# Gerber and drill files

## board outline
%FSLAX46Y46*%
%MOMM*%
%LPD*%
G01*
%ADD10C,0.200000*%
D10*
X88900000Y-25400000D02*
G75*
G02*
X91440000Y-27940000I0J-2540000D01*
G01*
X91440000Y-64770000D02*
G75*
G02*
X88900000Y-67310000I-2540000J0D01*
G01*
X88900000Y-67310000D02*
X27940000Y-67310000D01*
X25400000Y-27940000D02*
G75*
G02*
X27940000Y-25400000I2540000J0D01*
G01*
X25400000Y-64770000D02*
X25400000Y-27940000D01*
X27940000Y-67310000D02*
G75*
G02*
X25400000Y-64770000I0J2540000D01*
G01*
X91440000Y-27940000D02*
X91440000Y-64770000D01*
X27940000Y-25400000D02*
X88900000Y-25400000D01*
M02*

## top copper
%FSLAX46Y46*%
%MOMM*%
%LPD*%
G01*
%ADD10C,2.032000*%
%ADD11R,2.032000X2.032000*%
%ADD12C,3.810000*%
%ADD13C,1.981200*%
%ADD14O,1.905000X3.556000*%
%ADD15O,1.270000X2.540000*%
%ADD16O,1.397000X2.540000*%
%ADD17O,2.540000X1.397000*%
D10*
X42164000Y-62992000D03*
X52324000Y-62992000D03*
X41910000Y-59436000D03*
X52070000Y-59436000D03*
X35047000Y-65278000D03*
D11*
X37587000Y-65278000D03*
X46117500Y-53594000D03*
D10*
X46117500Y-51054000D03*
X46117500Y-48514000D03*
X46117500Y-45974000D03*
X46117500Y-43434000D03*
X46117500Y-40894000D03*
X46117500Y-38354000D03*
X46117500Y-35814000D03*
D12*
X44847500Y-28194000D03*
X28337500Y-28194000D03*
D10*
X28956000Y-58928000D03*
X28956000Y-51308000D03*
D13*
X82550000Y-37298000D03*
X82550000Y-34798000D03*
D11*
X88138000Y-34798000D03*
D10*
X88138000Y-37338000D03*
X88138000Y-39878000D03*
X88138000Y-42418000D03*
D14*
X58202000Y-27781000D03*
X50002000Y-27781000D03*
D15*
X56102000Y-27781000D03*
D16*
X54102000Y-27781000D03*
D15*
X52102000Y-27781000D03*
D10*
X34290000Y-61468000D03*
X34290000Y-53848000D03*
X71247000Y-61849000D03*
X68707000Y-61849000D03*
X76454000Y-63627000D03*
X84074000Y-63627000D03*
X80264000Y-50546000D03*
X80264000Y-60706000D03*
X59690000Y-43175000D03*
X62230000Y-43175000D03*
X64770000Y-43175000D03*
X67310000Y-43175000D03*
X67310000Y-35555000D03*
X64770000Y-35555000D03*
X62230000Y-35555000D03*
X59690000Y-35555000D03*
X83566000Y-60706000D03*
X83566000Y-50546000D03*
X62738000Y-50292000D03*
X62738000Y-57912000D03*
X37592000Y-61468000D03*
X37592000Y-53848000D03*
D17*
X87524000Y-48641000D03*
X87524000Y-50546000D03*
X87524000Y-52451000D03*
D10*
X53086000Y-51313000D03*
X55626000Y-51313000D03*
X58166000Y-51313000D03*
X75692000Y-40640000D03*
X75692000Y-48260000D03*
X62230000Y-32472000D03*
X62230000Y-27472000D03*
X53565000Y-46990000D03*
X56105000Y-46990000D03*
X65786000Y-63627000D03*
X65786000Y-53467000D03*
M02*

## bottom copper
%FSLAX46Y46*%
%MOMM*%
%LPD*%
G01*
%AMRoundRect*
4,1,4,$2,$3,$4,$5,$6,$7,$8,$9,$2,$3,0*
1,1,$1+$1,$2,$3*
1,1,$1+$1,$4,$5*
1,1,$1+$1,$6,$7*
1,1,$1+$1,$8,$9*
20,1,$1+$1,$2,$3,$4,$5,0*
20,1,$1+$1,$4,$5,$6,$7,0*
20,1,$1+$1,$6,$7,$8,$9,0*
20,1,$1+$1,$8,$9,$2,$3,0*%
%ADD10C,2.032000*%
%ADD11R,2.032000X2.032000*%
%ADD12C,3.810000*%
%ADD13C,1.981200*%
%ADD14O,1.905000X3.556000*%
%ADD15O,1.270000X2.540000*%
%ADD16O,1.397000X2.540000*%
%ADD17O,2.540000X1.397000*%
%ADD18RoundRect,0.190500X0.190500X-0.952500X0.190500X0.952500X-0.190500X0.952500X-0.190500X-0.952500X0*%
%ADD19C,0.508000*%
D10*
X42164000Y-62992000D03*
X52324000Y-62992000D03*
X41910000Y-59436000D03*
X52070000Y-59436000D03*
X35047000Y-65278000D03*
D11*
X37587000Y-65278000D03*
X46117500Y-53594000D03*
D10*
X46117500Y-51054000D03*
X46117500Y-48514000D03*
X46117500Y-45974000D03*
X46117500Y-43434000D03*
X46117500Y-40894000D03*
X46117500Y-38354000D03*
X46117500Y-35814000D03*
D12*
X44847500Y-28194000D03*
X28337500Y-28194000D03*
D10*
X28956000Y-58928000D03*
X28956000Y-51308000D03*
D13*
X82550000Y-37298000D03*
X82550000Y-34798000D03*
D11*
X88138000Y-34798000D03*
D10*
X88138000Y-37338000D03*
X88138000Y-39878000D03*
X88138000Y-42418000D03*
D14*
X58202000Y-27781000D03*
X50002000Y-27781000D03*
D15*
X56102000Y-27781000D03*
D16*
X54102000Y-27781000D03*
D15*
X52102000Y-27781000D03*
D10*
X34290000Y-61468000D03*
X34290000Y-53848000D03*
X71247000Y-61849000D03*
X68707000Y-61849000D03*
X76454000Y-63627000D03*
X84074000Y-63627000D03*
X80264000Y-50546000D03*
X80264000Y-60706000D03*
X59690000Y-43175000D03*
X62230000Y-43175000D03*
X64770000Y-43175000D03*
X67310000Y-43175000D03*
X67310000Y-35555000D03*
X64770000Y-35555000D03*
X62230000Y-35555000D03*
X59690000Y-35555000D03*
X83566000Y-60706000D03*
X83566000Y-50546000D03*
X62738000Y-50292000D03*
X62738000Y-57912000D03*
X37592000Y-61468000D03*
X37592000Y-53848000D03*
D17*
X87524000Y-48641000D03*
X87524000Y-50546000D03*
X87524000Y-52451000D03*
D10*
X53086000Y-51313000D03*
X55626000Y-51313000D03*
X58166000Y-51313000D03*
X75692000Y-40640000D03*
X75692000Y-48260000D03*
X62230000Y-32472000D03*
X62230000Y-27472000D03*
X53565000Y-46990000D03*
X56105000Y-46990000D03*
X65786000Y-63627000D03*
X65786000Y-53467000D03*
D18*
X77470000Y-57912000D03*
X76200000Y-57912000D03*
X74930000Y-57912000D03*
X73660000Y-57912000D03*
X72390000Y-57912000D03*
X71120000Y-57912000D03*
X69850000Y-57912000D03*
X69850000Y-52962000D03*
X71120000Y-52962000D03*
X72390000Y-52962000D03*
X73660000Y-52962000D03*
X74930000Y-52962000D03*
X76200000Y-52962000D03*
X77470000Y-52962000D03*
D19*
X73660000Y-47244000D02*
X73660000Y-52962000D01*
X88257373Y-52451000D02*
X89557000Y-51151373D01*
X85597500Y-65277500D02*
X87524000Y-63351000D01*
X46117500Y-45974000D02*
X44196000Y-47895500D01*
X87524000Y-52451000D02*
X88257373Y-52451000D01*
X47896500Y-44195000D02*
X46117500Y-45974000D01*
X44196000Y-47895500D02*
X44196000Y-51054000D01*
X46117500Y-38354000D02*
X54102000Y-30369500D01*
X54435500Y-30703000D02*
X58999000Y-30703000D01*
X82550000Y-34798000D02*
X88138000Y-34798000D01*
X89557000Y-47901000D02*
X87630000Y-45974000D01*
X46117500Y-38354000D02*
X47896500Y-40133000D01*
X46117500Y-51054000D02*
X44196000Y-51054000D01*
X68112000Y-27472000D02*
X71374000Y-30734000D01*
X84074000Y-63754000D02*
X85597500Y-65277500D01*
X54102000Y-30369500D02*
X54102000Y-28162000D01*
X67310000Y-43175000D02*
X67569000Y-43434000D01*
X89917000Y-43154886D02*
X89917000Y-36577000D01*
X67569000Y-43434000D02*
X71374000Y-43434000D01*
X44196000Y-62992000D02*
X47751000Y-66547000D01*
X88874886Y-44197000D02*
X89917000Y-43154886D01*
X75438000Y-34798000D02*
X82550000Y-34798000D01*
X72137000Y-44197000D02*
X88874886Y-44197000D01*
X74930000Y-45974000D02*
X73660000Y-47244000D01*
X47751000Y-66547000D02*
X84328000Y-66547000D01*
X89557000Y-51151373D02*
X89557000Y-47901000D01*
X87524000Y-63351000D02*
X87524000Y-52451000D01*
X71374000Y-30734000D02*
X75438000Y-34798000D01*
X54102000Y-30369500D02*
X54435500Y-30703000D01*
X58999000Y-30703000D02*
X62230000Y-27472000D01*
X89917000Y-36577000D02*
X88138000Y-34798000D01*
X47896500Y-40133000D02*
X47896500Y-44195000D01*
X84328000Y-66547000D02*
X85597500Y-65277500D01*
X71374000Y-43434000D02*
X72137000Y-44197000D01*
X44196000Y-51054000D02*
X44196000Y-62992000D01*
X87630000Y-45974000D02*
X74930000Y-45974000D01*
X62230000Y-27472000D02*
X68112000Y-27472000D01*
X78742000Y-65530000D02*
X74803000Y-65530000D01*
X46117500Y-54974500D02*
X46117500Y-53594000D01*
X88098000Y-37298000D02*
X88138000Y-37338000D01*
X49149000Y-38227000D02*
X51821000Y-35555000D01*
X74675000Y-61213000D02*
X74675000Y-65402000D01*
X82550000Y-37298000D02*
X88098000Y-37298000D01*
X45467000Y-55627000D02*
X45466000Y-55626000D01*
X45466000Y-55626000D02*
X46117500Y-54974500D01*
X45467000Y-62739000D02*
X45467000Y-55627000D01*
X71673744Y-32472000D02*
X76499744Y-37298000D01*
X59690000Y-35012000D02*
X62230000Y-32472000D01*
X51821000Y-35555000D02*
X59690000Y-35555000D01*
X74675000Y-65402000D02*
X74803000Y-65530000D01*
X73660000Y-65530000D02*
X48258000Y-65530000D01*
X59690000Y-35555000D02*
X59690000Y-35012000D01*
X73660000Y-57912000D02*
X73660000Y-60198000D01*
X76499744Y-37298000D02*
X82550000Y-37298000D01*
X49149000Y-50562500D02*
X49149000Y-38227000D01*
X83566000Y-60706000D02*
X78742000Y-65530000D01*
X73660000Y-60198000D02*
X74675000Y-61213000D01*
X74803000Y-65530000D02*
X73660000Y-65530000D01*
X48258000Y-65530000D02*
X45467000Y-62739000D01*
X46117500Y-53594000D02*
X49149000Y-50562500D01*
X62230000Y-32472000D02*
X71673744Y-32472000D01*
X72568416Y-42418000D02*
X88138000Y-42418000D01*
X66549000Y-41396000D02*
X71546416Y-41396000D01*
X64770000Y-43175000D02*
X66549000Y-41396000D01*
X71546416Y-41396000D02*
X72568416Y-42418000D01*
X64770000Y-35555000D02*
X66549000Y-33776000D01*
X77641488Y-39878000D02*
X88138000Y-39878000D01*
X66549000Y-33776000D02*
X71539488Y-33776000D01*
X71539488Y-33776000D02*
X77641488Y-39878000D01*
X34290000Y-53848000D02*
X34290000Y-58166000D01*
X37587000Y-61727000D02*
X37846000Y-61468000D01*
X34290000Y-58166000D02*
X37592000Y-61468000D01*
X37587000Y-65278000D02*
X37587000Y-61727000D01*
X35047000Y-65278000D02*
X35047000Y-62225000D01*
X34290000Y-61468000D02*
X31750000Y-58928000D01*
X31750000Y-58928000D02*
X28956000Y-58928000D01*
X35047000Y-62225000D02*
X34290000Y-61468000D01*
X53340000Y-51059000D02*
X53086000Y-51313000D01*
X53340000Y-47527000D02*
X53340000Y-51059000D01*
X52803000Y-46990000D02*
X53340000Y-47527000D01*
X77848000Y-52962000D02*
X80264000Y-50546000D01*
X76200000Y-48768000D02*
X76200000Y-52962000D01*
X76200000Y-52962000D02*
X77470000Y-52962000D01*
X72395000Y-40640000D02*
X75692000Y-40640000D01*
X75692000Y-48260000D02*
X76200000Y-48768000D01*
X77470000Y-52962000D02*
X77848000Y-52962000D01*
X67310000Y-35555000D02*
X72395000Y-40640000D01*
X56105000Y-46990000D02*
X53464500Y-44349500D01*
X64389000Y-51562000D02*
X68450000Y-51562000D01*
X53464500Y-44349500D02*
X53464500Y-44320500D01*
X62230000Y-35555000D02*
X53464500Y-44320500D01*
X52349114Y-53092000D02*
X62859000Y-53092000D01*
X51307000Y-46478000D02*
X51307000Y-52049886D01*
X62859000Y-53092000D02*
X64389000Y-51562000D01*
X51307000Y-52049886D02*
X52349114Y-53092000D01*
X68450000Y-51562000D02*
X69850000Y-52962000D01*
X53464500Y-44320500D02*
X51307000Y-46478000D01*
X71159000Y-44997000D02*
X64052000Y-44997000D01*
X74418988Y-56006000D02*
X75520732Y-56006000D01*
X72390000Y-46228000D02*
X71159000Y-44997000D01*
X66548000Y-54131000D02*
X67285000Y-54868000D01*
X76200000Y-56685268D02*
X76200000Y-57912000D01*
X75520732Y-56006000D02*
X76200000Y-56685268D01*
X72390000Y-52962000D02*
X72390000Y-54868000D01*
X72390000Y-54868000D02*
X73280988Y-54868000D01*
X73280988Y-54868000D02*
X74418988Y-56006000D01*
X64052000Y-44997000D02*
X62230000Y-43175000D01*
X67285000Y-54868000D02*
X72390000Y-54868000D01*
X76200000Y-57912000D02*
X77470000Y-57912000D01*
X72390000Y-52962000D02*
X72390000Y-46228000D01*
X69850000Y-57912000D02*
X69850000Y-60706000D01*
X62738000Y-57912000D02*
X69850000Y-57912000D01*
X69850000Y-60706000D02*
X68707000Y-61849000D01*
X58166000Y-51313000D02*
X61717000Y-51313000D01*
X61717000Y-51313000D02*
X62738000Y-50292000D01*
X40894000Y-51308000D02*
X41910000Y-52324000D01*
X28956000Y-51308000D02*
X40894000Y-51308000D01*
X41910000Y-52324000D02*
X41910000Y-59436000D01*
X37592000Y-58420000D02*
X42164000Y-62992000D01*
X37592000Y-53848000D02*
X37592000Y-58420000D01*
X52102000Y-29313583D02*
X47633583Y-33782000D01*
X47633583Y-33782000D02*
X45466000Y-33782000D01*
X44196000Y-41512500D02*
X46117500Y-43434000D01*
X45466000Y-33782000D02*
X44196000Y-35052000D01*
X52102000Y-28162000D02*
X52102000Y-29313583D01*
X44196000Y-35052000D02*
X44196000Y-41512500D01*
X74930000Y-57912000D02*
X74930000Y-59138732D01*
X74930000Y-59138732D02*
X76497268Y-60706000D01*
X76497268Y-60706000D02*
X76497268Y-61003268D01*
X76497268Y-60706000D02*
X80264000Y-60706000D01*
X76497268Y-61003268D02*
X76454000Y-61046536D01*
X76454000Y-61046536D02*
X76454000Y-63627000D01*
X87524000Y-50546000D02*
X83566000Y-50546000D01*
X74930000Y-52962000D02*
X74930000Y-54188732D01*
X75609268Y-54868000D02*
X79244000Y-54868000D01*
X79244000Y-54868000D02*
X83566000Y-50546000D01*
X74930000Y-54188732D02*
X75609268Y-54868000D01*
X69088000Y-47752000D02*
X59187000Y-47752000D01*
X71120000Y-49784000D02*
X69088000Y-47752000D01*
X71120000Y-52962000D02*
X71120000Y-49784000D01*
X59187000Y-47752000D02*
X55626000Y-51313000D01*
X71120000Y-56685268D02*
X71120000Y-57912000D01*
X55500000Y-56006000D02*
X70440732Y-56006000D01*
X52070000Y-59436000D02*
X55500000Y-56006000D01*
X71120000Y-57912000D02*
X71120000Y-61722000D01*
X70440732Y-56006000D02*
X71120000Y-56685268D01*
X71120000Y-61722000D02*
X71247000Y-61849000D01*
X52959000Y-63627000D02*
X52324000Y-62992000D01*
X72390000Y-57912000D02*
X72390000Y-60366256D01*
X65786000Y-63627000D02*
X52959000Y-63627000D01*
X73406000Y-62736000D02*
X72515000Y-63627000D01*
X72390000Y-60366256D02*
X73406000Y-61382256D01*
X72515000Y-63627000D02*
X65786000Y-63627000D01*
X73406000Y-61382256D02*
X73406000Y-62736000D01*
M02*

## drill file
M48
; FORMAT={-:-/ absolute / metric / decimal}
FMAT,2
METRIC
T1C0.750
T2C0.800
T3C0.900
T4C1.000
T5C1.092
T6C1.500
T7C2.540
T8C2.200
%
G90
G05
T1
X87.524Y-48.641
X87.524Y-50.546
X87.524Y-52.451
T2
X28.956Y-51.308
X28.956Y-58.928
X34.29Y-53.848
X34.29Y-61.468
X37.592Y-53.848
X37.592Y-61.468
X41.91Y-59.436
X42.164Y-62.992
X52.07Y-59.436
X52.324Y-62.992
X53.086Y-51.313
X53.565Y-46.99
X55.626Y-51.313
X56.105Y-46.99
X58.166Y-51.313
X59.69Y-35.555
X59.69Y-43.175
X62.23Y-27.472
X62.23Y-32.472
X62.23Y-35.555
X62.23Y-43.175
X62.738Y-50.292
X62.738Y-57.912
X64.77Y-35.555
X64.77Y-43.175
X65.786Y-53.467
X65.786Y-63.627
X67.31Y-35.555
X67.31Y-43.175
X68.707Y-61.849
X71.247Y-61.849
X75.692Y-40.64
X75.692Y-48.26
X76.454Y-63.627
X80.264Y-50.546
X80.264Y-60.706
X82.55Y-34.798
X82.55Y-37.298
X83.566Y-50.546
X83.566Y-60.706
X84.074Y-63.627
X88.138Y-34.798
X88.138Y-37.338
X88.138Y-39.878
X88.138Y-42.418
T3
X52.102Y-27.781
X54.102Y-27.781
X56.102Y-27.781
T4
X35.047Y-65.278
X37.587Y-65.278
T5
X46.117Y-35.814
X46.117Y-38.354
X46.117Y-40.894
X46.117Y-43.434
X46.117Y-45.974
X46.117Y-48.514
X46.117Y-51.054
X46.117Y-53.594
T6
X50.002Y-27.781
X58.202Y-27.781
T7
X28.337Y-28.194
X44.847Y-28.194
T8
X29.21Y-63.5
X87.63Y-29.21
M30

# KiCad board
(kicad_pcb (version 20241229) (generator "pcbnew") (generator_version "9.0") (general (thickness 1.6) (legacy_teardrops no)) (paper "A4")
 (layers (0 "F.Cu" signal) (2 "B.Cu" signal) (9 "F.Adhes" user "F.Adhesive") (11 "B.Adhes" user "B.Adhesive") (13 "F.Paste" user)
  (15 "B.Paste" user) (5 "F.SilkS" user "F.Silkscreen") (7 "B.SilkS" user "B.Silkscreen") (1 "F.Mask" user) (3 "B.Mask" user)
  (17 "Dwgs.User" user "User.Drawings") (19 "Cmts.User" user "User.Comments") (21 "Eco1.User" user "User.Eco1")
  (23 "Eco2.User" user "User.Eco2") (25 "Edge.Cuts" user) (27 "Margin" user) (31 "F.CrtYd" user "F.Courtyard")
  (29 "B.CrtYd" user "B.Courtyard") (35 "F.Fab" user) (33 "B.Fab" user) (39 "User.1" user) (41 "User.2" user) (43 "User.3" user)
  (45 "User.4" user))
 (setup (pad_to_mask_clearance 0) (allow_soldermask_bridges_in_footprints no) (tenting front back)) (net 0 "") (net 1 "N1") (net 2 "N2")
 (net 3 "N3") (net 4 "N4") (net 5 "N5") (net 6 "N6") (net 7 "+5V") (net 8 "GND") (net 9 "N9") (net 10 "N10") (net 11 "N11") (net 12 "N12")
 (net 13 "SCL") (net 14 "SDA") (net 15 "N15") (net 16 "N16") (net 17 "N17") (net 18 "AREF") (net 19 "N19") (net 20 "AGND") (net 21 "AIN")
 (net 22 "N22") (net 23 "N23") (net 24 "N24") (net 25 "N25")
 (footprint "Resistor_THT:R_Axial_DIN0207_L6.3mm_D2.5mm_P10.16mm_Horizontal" (layer "F.Cu") (at 42.164 62.992)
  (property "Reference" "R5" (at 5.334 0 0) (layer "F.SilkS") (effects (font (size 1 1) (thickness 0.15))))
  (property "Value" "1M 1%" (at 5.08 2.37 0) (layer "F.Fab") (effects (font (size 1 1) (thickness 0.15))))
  (pad "1" thru_hole circle (at 0 0) (size 2.032 2.032) (drill 0.8) (layers "*.Cu" "*.Mask") (remove_unused_layers no) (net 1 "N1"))
  (pad "2" thru_hole circle (at 10.16 0) (size 2.032 2.032) (drill 0.8) (layers "*.Cu" "*.Mask") (remove_unused_layers no) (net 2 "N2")))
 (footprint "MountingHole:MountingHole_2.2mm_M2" (layer "F.Cu") (at 29.21 63.5)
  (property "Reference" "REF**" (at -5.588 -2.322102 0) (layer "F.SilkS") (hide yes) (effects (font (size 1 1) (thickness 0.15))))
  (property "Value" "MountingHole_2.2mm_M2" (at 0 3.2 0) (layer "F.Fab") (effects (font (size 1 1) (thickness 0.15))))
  (pad "" np_thru_hole circle (at 0 0) (size 2.2 2.2) (drill 2.2) (layers "*.Cu" "*.Mask")))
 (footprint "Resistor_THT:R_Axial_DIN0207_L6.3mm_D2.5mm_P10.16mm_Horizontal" (layer "F.Cu") (at 41.91 59.436)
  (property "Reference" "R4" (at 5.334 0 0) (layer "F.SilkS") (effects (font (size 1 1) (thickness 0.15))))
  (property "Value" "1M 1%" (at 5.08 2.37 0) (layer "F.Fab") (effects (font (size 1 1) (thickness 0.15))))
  (pad "1" thru_hole circle (at 0 0) (size 2.032 2.032) (drill 0.8) (layers "*.Cu" "*.Mask") (remove_unused_layers no) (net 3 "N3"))
  (pad "2" thru_hole circle (at 10.16 0) (size 2.032 2.032) (drill 0.8) (layers "*.Cu" "*.Mask") (remove_unused_layers no) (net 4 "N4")))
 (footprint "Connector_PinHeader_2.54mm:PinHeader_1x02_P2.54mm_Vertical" (layer "F.Cu") (at 35.047 65.278 90)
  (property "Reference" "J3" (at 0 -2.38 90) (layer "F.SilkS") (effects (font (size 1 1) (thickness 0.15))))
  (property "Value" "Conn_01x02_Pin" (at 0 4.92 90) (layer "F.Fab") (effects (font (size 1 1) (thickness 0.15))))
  (pad "1" thru_hole circle (at 0 0 90) (size 2.032 2.032) (drill 1) (layers "*.Cu" "*.Mask") (remove_unused_layers no) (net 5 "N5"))
  (pad "2" thru_hole rect (at 0 2.54 90) (size 2.032 2.032) (drill 1) (layers "*.Cu" "*.Mask") (remove_unused_layers no) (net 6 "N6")))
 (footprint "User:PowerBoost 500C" (layer "F.Cu") (at 46.1175 53.594 180)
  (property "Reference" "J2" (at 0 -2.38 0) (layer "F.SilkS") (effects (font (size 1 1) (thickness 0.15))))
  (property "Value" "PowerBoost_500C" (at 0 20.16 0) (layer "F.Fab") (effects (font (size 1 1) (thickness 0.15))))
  (pad "1" thru_hole rect (at 0 0 180) (size 2.032 2.032) (drill 1.0922) (layers "*.Cu" "*.Mask") (remove_unused_layers no) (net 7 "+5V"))
  (pad "2" thru_hole circle (at 0 2.54 180) (size 2.032 2.032) (drill 1.0922) (layers "*.Cu" "*.Mask") (remove_unused_layers no)
   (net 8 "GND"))
  (pad "3" thru_hole circle (at 0 5.08 180) (size 2.032 2.032) (drill 1.0922) (layers "*.Cu" "*.Mask") (remove_unused_layers no)
   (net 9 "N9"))
  (pad "4" thru_hole circle (at 0 7.62 180) (size 2.032 2.032) (drill 1.0922) (layers "*.Cu" "*.Mask") (remove_unused_layers no)
   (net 8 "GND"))
  (pad "5" thru_hole circle (at 0 10.16 180) (size 2.032 2.032) (drill 1.0922) (layers "*.Cu" "*.Mask") (remove_unused_layers no)
   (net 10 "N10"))
  (pad "6" thru_hole circle (at 0 12.7 180) (size 2.032 2.032) (drill 1.0922) (layers "*.Cu" "*.Mask") (remove_unused_layers no)
   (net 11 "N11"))
  (pad "7" thru_hole circle (at 0 15.24 180) (size 2.032 2.032) (drill 1.0922) (layers "*.Cu" "*.Mask") (remove_unused_layers no)
   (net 8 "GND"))
  (pad "8" thru_hole circle (at 0 17.78 180) (size 2.032 2.032) (drill 1.0922) (layers "*.Cu" "*.Mask") (remove_unused_layers no)
   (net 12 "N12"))
  (pad "9" thru_hole circle (at 1.27 25.4 180) (size 3.81 3.81) (drill 2.54) (layers "*.Cu" "*.Mask") (remove_unused_layers no))
  (pad "9" thru_hole circle (at 17.78 25.4 180) (size 3.81 3.81) (drill 2.54) (layers "*.Cu" "*.Mask") (remove_unused_layers no)))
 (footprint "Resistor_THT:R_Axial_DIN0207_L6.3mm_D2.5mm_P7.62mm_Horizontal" (layer "F.Cu") (at 28.956 58.928 90)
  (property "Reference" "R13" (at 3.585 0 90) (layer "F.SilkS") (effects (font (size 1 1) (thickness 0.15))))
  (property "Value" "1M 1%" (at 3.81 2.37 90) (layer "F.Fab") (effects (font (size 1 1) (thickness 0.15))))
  (pad "1" thru_hole circle (at 0 0 90) (size 2.032 2.032) (drill 0.8) (layers "*.Cu" "*.Mask") (remove_unused_layers no) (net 5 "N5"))
  (pad "2" thru_hole circle (at 7.62 0 90) (size 2.032 2.032) (drill 0.8) (layers "*.Cu" "*.Mask") (remove_unused_layers no) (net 3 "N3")))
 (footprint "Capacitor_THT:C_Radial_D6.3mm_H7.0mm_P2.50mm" (layer "F.Cu") (at 82.55 37.298 90)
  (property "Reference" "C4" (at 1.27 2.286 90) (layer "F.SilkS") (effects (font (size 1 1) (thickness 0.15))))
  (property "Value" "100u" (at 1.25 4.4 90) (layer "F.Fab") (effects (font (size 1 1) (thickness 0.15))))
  (pad "1" thru_hole circle (at 0 0 90) (size 1.9812 1.9812) (drill 0.8) (layers "*.Cu" "*.Mask") (remove_unused_layers no) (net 7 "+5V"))
  (pad "2" thru_hole circle (at 2.5 0 90) (size 1.9812 1.9812) (drill 0.8) (layers "*.Cu" "*.Mask") (remove_unused_layers no) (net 8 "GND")))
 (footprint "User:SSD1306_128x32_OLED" (layer "F.Cu") (at 88.138 34.798)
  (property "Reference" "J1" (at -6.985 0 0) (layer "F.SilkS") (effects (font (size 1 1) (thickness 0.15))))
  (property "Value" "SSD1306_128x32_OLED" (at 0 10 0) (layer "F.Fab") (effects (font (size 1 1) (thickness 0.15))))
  (pad "1" thru_hole rect (at 0 0) (size 2.032 2.032) (drill 0.8) (layers "*.Cu" "*.Mask") (remove_unused_layers no) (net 8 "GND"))
  (pad "2" thru_hole circle (at 0 2.54) (size 2.032 2.032) (drill 0.8) (layers "*.Cu" "*.Mask") (remove_unused_layers no) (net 7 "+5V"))
  (pad "3" thru_hole circle (at 0 5.08) (size 2.032 2.032) (drill 0.8) (layers "*.Cu" "*.Mask") (remove_unused_layers no) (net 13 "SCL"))
  (pad "4" thru_hole circle (at 0 7.62) (size 2.032 2.032) (drill 0.8) (layers "*.Cu" "*.Mask") (remove_unused_layers no) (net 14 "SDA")))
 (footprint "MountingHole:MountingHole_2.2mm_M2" (layer "F.Cu") (at 87.63 29.21)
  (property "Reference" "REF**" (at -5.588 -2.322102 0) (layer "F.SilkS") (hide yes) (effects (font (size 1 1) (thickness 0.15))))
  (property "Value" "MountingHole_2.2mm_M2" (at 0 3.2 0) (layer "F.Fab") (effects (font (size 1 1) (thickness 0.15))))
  (pad "" np_thru_hole circle (at 0 0) (size 2.2 2.2) (drill 2.2) (layers "*.Cu" "*.Mask")))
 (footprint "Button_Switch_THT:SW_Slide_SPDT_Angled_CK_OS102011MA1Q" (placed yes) (layer "F.Cu") (at 56.102 27.781 180)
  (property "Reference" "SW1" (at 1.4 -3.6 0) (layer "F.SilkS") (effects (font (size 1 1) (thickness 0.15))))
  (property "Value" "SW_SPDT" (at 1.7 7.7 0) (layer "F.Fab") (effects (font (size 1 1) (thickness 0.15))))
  (pad "" thru_hole oval (at -2.1 0 180) (size 1.905 3.556) (drill 1.5) (layers "*.Cu" "*.Mask") (remove_unused_layers no))
  (pad "" thru_hole oval (at 6.1 0 180) (size 1.905 3.556) (drill 1.5) (layers "*.Cu" "*.Mask") (remove_unused_layers no))
  (pad "1" thru_hole oval (at 0 0 180) (size 1.27 2.54) (drill 0.9) (layers "*.Cu" "*.Mask") (remove_unused_layers no) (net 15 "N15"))
  (pad "2" thru_hole oval (at 2 0 180) (size 1.397 2.54) (drill 0.9) (layers "*.Cu" "*.Mask") (remove_unused_layers no) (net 8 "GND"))
  (pad "3" thru_hole oval (at 4 0 180) (size 1.27 2.54) (drill 0.9) (layers "*.Cu" "*.Mask") (remove_unused_layers no) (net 10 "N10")))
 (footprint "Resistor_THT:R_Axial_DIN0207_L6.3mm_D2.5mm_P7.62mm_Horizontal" (layer "F.Cu") (at 34.29 61.468 90)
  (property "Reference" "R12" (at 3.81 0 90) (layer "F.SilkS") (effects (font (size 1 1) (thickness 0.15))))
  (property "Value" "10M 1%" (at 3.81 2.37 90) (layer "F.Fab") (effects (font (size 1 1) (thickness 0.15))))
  (pad "1" thru_hole circle (at 0 0 90) (size 2.032 2.032) (drill 0.8) (layers "*.Cu" "*.Mask") (remove_unused_layers no) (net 5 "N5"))
  (pad "2" thru_hole circle (at 7.62 0 90) (size 2.032 2.032) (drill 0.8) (layers "*.Cu" "*.Mask") (remove_unused_layers no) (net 6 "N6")))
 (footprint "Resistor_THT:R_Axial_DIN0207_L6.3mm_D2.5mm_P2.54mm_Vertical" (layer "F.Cu") (at 71.247 61.849 180)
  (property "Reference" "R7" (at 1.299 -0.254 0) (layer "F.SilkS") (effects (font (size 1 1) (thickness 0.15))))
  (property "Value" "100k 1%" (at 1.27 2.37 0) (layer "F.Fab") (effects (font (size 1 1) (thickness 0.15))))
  (pad "1" thru_hole circle (at 0 0 180) (size 2.032 2.032) (drill 0.8) (layers "*.Cu" "*.Mask") (remove_unused_layers no) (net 4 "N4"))
  (pad "2" thru_hole circle (at 2.54 0 180) (size 2.032 2.032) (drill 0.8) (layers "*.Cu" "*.Mask") (remove_unused_layers no) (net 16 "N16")))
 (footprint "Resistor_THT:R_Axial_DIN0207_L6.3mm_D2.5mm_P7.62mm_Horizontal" (layer "F.Cu") (at 76.454 63.627)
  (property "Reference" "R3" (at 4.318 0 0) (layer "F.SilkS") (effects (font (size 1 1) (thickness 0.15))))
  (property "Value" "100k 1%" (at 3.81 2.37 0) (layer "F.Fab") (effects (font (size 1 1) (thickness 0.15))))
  (pad "1" thru_hole circle (at 0 0) (size 2.032 2.032) (drill 0.8) (layers "*.Cu" "*.Mask") (remove_unused_layers no) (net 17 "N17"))
  (pad "2" thru_hole circle (at 7.62 0) (size 2.032 2.032) (drill 0.8) (layers "*.Cu" "*.Mask") (remove_unused_layers no) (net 8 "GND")))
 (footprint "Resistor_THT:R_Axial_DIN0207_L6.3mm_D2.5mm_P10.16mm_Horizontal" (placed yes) (layer "F.Cu") (at 80.264 50.546 -90)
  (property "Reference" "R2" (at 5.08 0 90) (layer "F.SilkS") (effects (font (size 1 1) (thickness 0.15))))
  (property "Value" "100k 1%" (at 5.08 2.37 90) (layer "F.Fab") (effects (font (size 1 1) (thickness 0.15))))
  (pad "1" thru_hole circle (at 0 0 270) (size 2.032 2.032) (drill 0.8) (layers "*.Cu" "*.Mask") (remove_unused_layers no) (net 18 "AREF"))
  (pad "2" thru_hole circle (at 10.16 0 270) (size 2.032 2.032) (drill 0.8) (layers "*.Cu" "*.Mask") (remove_unused_layers no)
   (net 17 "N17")))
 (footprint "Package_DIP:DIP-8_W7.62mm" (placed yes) (layer "F.Cu") (at 59.69 43.175 90)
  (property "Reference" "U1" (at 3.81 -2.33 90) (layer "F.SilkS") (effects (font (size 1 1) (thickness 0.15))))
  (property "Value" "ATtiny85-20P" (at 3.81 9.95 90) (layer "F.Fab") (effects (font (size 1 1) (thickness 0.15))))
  (pad "1" thru_hole circle (at 0 0 90) (size 2.032 2.032) (drill 0.8) (layers "*.Cu" "*.Mask") (remove_unused_layers no) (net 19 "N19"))
  (pad "2" thru_hole circle (at 0 2.54 90) (size 2.032 2.032) (drill 0.8) (layers "*.Cu" "*.Mask") (remove_unused_layers no) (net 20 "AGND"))
  (pad "3" thru_hole circle (at 0 5.08 90) (size 2.032 2.032) (drill 0.8) (layers "*.Cu" "*.Mask") (remove_unused_layers no) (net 14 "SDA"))
  (pad "4" thru_hole circle (at 0 7.62 90) (size 2.032 2.032) (drill 0.8) (layers "*.Cu" "*.Mask") (remove_unused_layers no) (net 8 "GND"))
  (pad "5" thru_hole circle (at 7.62 7.62 90) (size 2.032 2.032) (drill 0.8) (layers "*.Cu" "*.Mask") (remove_unused_layers no)
   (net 18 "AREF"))
  (pad "6" thru_hole circle (at 7.62 5.08 90) (size 2.032 2.032) (drill 0.8) (layers "*.Cu" "*.Mask") (remove_unused_layers no)
   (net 13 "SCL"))
  (pad "7" thru_hole circle (at 7.62 2.54 90) (size 2.032 2.032) (drill 0.8) (layers "*.Cu" "*.Mask") (remove_unused_layers no)
   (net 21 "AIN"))
  (pad "8" thru_hole circle (at 7.62 0 90) (size 2.032 2.032) (drill 0.8) (layers "*.Cu" "*.Mask") (remove_unused_layers no) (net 7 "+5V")))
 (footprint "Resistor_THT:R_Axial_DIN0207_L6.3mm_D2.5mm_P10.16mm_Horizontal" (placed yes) (layer "F.Cu") (at 83.566 60.706 90)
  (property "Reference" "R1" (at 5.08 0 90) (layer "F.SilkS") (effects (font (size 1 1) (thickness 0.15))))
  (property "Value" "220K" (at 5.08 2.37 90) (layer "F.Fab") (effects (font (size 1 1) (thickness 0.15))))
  (pad "1" thru_hole circle (at 0 0 90) (size 2.032 2.032) (drill 0.8) (layers "*.Cu" "*.Mask") (remove_unused_layers no) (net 7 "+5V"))
  (pad "2" thru_hole circle (at 10.16 0 90) (size 2.032 2.032) (drill 0.8) (layers "*.Cu" "*.Mask") (remove_unused_layers no) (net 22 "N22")))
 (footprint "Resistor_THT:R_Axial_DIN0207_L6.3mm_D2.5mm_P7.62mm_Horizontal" (layer "F.Cu") (at 62.738 50.292 -90)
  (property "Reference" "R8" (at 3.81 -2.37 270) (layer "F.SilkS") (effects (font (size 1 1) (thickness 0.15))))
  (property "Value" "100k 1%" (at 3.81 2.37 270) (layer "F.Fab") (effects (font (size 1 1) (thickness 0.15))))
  (pad "1" thru_hole circle (at 0 0 270) (size 2.032 2.032) (drill 0.8) (layers "*.Cu" "*.Mask") (remove_unused_layers no) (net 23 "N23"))
  (pad "2" thru_hole circle (at 7.62 0 270) (size 2.032 2.032) (drill 0.8) (layers "*.Cu" "*.Mask") (remove_unused_layers no) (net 16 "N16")))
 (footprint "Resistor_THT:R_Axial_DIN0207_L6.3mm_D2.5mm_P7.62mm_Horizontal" (layer "F.Cu") (at 37.592 61.468 90)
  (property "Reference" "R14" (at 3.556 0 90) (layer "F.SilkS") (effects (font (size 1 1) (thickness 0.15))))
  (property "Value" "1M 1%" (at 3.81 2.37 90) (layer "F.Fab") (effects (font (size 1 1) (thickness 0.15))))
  (pad "1" thru_hole circle (at 0 0 90) (size 2.032 2.032) (drill 0.8) (layers "*.Cu" "*.Mask") (remove_unused_layers no) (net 6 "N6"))
  (pad "2" thru_hole circle (at 7.62 0 90) (size 2.032 2.032) (drill 0.8) (layers "*.Cu" "*.Mask") (remove_unused_layers no) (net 1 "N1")))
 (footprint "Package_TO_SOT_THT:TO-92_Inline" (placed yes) (layer "F.Cu") (at 87.524 49.276 -90)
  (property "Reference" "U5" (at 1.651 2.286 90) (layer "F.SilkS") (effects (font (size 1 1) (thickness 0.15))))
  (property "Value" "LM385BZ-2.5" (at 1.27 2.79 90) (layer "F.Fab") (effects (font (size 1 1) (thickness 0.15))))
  (pad "1" thru_hole oval (at -0.635 0 270) (size 1.397 2.54) (drill 0.75) (layers "*.Cu" "*.Mask") (remove_unused_layers no))
  (pad "2" thru_hole oval (at 1.27 0 270) (size 1.397 2.54) (drill 0.75) (layers "*.Cu" "*.Mask") (remove_unused_layers no) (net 22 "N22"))
  (pad "3" thru_hole oval (at 3.175 0 270) (size 1.397 2.54) (drill 0.75) (layers "*.Cu" "*.Mask") (remove_unused_layers no) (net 8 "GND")))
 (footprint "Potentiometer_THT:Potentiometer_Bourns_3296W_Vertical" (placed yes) (layer "F.Cu") (at 53.086 51.313 180)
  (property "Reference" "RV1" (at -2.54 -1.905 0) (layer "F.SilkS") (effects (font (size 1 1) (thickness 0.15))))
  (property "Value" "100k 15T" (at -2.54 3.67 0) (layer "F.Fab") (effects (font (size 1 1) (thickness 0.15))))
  (pad "1" thru_hole circle (at 0 0 180) (size 2.032 2.032) (drill 0.8) (layers "*.Cu" "*.Mask") (remove_unused_layers no) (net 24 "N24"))
  (pad "2" thru_hole circle (at -2.54 0 180) (size 2.032 2.032) (drill 0.8) (layers "*.Cu" "*.Mask") (remove_unused_layers no)
   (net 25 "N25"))
  (pad "3" thru_hole circle (at -5.08 0 180) (size 2.032 2.032) (drill 0.8) (layers "*.Cu" "*.Mask") (remove_unused_layers no)
   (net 23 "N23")))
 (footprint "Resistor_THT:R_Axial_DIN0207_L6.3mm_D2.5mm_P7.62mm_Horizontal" (layer "F.Cu") (at 75.692 40.64 -90)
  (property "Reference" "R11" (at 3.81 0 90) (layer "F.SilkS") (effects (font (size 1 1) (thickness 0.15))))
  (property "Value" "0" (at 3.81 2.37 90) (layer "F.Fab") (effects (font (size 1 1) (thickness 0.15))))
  (pad "1" thru_hole circle (at 0 0 270) (size 2.032 2.032) (drill 0.8) (layers "*.Cu" "*.Mask") (remove_unused_layers no) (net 18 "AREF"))
  (pad "2" thru_hole circle (at 7.62 0 270) (size 2.032 2.032) (drill 0.8) (layers "*.Cu" "*.Mask") (remove_unused_layers no)
   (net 18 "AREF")))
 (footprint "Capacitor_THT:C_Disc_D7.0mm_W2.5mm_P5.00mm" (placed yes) (layer "F.Cu") (at 62.23 32.472 90)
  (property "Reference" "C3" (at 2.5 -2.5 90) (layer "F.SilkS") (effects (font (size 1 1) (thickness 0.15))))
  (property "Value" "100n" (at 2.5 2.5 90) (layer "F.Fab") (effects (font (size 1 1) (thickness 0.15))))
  (pad "1" thru_hole circle (at 0 0 90) (size 2.032 2.032) (drill 0.8) (layers "*.Cu" "*.Mask") (remove_unused_layers no) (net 7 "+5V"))
  (pad "2" thru_hole circle (at 5 0 90) (size 2.032 2.032) (drill 0.8) (layers "*.Cu" "*.Mask") (remove_unused_layers no) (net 8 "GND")))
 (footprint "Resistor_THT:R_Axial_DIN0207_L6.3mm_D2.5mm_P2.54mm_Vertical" (layer "F.Cu") (at 53.565 46.99)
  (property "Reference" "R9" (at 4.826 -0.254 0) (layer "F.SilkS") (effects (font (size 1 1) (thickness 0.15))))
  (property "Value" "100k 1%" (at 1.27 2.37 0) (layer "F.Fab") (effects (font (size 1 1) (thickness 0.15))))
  (pad "1" thru_hole circle (at 0 0) (size 2.032 2.032) (drill 0.8) (layers "*.Cu" "*.Mask") (remove_unused_layers no) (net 24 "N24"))
  (pad "2" thru_hole circle (at 2.54 0) (size 2.032 2.032) (drill 0.8) (layers "*.Cu" "*.Mask") (remove_unused_layers no) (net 21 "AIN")))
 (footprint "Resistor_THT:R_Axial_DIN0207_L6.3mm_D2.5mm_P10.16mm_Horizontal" (layer "F.Cu") (at 65.786 63.627 90)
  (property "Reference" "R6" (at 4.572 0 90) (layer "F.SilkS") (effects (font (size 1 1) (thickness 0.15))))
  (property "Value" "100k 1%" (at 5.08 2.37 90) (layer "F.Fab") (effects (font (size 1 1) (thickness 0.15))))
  (pad "1" thru_hole circle (at 0 0 90) (size 2.032 2.032) (drill 0.8) (layers "*.Cu" "*.Mask") (remove_unused_layers no) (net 2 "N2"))
  (pad "2" thru_hole circle (at 10.16 0 90) (size 2.032 2.032) (drill 0.8) (layers "*.Cu" "*.Mask") (remove_unused_layers no)
   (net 20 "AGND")))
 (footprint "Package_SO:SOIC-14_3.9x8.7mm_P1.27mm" (layer "B.Cu") (at 73.66 55.437 90)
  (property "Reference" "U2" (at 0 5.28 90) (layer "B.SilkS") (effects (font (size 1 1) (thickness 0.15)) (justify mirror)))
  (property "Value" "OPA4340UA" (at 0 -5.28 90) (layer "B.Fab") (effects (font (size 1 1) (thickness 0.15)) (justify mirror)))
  (pad "1" smd roundrect (at -2.475 3.81 90) (size 2.286 0.762) (layers "B.Cu" "B.Mask" "B.Paste") (roundrect_rratio 0.25) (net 20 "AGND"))
  (pad "2" smd roundrect (at -2.475 2.54 90) (size 2.286 0.762) (layers "B.Cu" "B.Mask" "B.Paste") (roundrect_rratio 0.25) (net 20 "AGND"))
  (pad "3" smd roundrect (at -2.475 1.27 90) (size 2.286 0.762) (layers "B.Cu" "B.Mask" "B.Paste") (roundrect_rratio 0.25) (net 17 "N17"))
  (pad "4" smd roundrect (at -2.475 0 90) (size 2.286 0.762) (layers "B.Cu" "B.Mask" "B.Paste") (roundrect_rratio 0.25) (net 7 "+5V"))
  (pad "5" smd roundrect (at -2.475 -1.27 90) (size 2.286 0.762) (layers "B.Cu" "B.Mask" "B.Paste") (roundrect_rratio 0.25) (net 2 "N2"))
  (pad "6" smd roundrect (at -2.475 -2.54 90) (size 2.286 0.762) (layers "B.Cu" "B.Mask" "B.Paste") (roundrect_rratio 0.25) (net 4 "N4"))
  (pad "7" smd roundrect (at -2.475 -3.81 90) (size 2.286 0.762) (layers "B.Cu" "B.Mask" "B.Paste") (roundrect_rratio 0.25) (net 16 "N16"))
  (pad "8" smd roundrect (at 2.475 -3.81 90) (size 2.286 0.762) (layers "B.Cu" "B.Mask" "B.Paste") (roundrect_rratio 0.25) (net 21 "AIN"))
  (pad "9" smd roundrect (at 2.475 -2.54 90) (size 2.286 0.762) (layers "B.Cu" "B.Mask" "B.Paste") (roundrect_rratio 0.25) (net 25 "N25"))
  (pad "10" smd roundrect (at 2.475 -1.27 90) (size 2.286 0.762) (layers "B.Cu" "B.Mask" "B.Paste") (roundrect_rratio 0.25) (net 20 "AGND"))
  (pad "11" smd roundrect (at 2.475 0 90) (size 2.286 0.762) (layers "B.Cu" "B.Mask" "B.Paste") (roundrect_rratio 0.25) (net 8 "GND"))
  (pad "12" smd roundrect (at 2.475 1.27 90) (size 2.286 0.762) (layers "B.Cu" "B.Mask" "B.Paste") (roundrect_rratio 0.25) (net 22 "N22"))
  (pad "13" smd roundrect (at 2.475 2.54 90) (size 2.286 0.762) (layers "B.Cu" "B.Mask" "B.Paste") (roundrect_rratio 0.25) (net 18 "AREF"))
  (pad "14" smd roundrect (at 2.475 3.81 90) (size 2.286 0.762) (layers "B.Cu" "B.Mask" "B.Paste") (roundrect_rratio 0.25) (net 18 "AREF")))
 (gr_arc (start 88.9 25.4) (mid 90.696051 26.143949) (end 91.44 27.94) (stroke (width 0.2) (type default)) (layer "Edge.Cuts"))
 (gr_arc (start 91.44 64.77) (mid 90.696051 66.566051) (end 88.9 67.31) (stroke (width 0.2) (type default)) (layer "Edge.Cuts"))
 (gr_line (start 88.9 67.31) (end 27.94 67.31) (stroke (width 0.2) (type default)) (layer "Edge.Cuts"))
 (gr_arc (start 25.4 27.94) (mid 26.143949 26.143949) (end 27.94 25.4) (stroke (width 0.2) (type default)) (layer "Edge.Cuts"))
 (gr_line (start 25.4 64.77) (end 25.4 27.94) (stroke (width 0.2) (type default)) (layer "Edge.Cuts"))
 (gr_arc (start 27.94 67.31) (mid 26.143949 66.566051) (end 25.4 64.77) (stroke (width 0.2) (type default)) (layer "Edge.Cuts"))
 (gr_line (start 91.44 27.94) (end 91.44 64.77) (stroke (width 0.2) (type default)) (layer "Edge.Cuts"))
 (gr_line (start 27.94 25.4) (end 88.9 25.4) (stroke (width 0.2) (type default)) (layer "Edge.Cuts"))
 (segment (start 73.66 47.244) (end 73.66 52.962) (width 0.508) (layer "B.Cu") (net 8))
 (segment (start 88.257373 52.451) (end 89.557 51.151373) (width 0.508) (layer "B.Cu") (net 8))
 (segment (start 85.5975 65.2775) (end 87.524 63.351) (width 0.508) (layer "B.Cu") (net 8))
 (segment (start 46.1175 45.974) (end 44.196 47.8955) (width 0.508) (layer "B.Cu") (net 8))
 (segment (start 87.524 52.451) (end 88.257373 52.451) (width 0.508) (layer "B.Cu") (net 8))
 (segment (start 47.8965 44.195) (end 46.1175 45.974) (width 0.508) (layer "B.Cu") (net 8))
 (segment (start 44.196 47.8955) (end 44.196 51.054) (width 0.508) (layer "B.Cu") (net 8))
 (segment (start 46.1175 38.354) (end 54.102 30.3695) (width 0.508) (layer "B.Cu") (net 8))
 (segment (start 54.4355 30.703) (end 58.999 30.703) (width 0.508) (layer "B.Cu") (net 8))
 (segment (start 82.55 34.798) (end 88.138 34.798) (width 0.508) (layer "B.Cu") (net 8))
 (segment (start 89.557 47.901) (end 87.63 45.974) (width 0.508) (layer "B.Cu") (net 8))
 (segment (start 46.1175 38.354) (end 47.8965 40.133) (width 0.508) (layer "B.Cu") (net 8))
 (segment (start 46.1175 51.054) (end 44.196 51.054) (width 0.508) (layer "B.Cu") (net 8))
 (segment (start 68.112 27.472) (end 71.374 30.734) (width 0.508) (layer "B.Cu") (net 8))
 (segment (start 84.074 63.754) (end 85.5975 65.2775) (width 0.508) (layer "B.Cu") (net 8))
 (segment (start 54.102 30.3695) (end 54.102 28.162) (width 0.508) (layer "B.Cu") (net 8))
 (segment (start 67.31 43.175) (end 67.569 43.434) (width 0.508) (layer "B.Cu") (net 8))
 (segment (start 89.917 43.154886) (end 89.917 36.577) (width 0.508) (layer "B.Cu") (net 8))
 (segment (start 67.569 43.434) (end 71.374 43.434) (width 0.508) (layer "B.Cu") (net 8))
 (segment (start 44.196 62.992) (end 47.751 66.547) (width 0.508) (layer "B.Cu") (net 8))
 (segment (start 88.874886 44.197) (end 89.917 43.154886) (width 0.508) (layer "B.Cu") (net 8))
 (segment (start 75.438 34.798) (end 82.55 34.798) (width 0.508) (layer "B.Cu") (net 8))
 (segment (start 72.137 44.197) (end 88.874886 44.197) (width 0.508) (layer "B.Cu") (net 8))
 (segment (start 74.93 45.974) (end 73.66 47.244) (width 0.508) (layer "B.Cu") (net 8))
 (segment (start 47.751 66.547) (end 84.328 66.547) (width 0.508) (layer "B.Cu") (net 8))
 (segment (start 89.557 51.151373) (end 89.557 47.901) (width 0.508) (layer "B.Cu") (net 8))
 (segment (start 87.524 63.351) (end 87.524 52.451) (width 0.508) (layer "B.Cu") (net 8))
 (segment (start 71.374 30.734) (end 75.438 34.798) (width 0.508) (layer "B.Cu") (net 8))
 (segment (start 54.102 30.3695) (end 54.4355 30.703) (width 0.508) (layer "B.Cu") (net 8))
 (segment (start 58.999 30.703) (end 62.23 27.472) (width 0.508) (layer "B.Cu") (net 8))
 (segment (start 89.917 36.577) (end 88.138 34.798) (width 0.508) (layer "B.Cu") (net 8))
 (segment (start 47.8965 40.133) (end 47.8965 44.195) (width 0.508) (layer "B.Cu") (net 8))
 (segment (start 84.328 66.547) (end 85.5975 65.2775) (width 0.508) (layer "B.Cu") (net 8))
 (segment (start 71.374 43.434) (end 72.137 44.197) (width 0.508) (layer "B.Cu") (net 8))
 (segment (start 44.196 51.054) (end 44.196 62.992) (width 0.508) (layer "B.Cu") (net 8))
 (segment (start 87.63 45.974) (end 74.93 45.974) (width 0.508) (layer "B.Cu") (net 8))
 (segment (start 62.23 27.472) (end 68.112 27.472) (width 0.508) (layer "B.Cu") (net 8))
 (segment (start 78.742 65.53) (end 74.803 65.53) (width 0.508) (layer "B.Cu") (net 7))
 (segment (start 46.1175 54.9745) (end 46.1175 53.594) (width 0.508) (layer "B.Cu") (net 7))
 (segment (start 88.098 37.298) (end 88.138 37.338) (width 0.508) (layer "B.Cu") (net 7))
 (segment (start 49.149 38.227) (end 51.821 35.555) (width 0.508) (layer "B.Cu") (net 7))
 (segment (start 74.675 61.213) (end 74.675 65.402) (width 0.508) (layer "B.Cu") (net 7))
 (segment (start 82.55 37.298) (end 88.098 37.298) (width 0.508) (layer "B.Cu") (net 7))
 (segment (start 45.467 55.627) (end 45.466 55.626) (width 0.508) (layer "B.Cu") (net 7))
 (segment (start 45.466 55.626) (end 46.1175 54.9745) (width 0.508) (layer "B.Cu") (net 7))
 (segment (start 45.467 62.739) (end 45.467 55.627) (width 0.508) (layer "B.Cu") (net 7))
 (segment (start 71.673744 32.472) (end 76.499744 37.298) (width 0.508) (layer "B.Cu") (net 7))
 (segment (start 59.69 35.012) (end 62.23 32.472) (width 0.508) (layer "B.Cu") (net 7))
 (segment (start 51.821 35.555) (end 59.69 35.555) (width 0.508) (layer "B.Cu") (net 7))
 (segment (start 74.675 65.402) (end 74.803 65.53) (width 0.508) (layer "B.Cu") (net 7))
 (segment (start 73.66 65.53) (end 48.258 65.53) (width 0.508) (layer "B.Cu") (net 7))
 (segment (start 59.69 35.555) (end 59.69 35.012) (width 0.508) (layer "B.Cu") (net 7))
 (segment (start 73.66 57.912) (end 73.66 60.198) (width 0.508) (layer "B.Cu") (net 7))
 (segment (start 76.499744 37.298) (end 82.55 37.298) (width 0.508) (layer "B.Cu") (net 7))
 (segment (start 49.149 50.5625) (end 49.149 38.227) (width 0.508) (layer "B.Cu") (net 7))
 (segment (start 83.566 60.706) (end 78.742 65.53) (width 0.508) (layer "B.Cu") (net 7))
 (segment (start 73.66 60.198) (end 74.675 61.213) (width 0.508) (layer "B.Cu") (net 7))
 (segment (start 74.803 65.53) (end 73.66 65.53) (width 0.508) (layer "B.Cu") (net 7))
 (segment (start 48.258 65.53) (end 45.467 62.739) (width 0.508) (layer "B.Cu") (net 7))
 (segment (start 46.1175 53.594) (end 49.149 50.5625) (width 0.508) (layer "B.Cu") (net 7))
 (segment (start 62.23 32.472) (end 71.673744 32.472) (width 0.508) (layer "B.Cu") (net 7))
 (segment (start 72.568416 42.418) (end 88.138 42.418) (width 0.508) (layer "B.Cu") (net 14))
 (segment (start 66.549 41.396) (end 71.546416 41.396) (width 0.508) (layer "B.Cu") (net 14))
 (segment (start 64.77 43.175) (end 66.549 41.396) (width 0.508) (layer "B.Cu") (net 14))
 (segment (start 71.546416 41.396) (end 72.568416 42.418) (width 0.508) (layer "B.Cu") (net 14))
 (segment (start 64.77 35.555) (end 66.549 33.776) (width 0.508) (layer "B.Cu") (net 13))
 (segment (start 77.641488 39.878) (end 88.138 39.878) (width 0.508) (layer "B.Cu") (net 13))
 (segment (start 66.549 33.776) (end 71.539488 33.776) (width 0.508) (layer "B.Cu") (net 13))
 (segment (start 71.539488 33.776) (end 77.641488 39.878) (width 0.508) (layer "B.Cu") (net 13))
 (segment (start 34.29 53.848) (end 34.29 58.166) (width 0.508) (layer "B.Cu") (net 6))
 (segment (start 37.587 61.727) (end 37.846 61.468) (width 0.508) (layer "B.Cu") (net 6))
 (segment (start 34.29 58.166) (end 37.592 61.468) (width 0.508) (layer "B.Cu") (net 6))
 (segment (start 37.587 65.278) (end 37.587 61.727) (width 0.508) (layer "B.Cu") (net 6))
 (segment (start 35.047 65.278) (end 35.047 62.225) (width 0.508) (layer "B.Cu") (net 5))
 (segment (start 34.29 61.468) (end 31.75 58.928) (width 0.508) (layer "B.Cu") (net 5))
 (segment (start 31.75 58.928) (end 28.956 58.928) (width 0.508) (layer "B.Cu") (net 5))
 (segment (start 35.047 62.225) (end 34.29 61.468) (width 0.508) (layer "B.Cu") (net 5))
 (segment (start 53.34 51.059) (end 53.086 51.313) (width 0.508) (layer "B.Cu") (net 24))
 (segment (start 53.34 47.527) (end 53.34 51.059) (width 0.508) (layer "B.Cu") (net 24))
 (segment (start 52.803 46.99) (end 53.34 47.527) (width 0.508) (layer "B.Cu") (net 24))
 (segment (start 77.848 52.962) (end 80.264 50.546) (width 0.508) (layer "B.Cu") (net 18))
 (segment (start 76.2 48.768) (end 76.2 52.962) (width 0.508) (layer "B.Cu") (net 18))
 (segment (start 76.2 52.962) (end 77.47 52.962) (width 0.508) (layer "B.Cu") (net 18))
 (segment (start 72.395 40.64) (end 75.692 40.64) (width 0.508) (layer "B.Cu") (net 18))
 (segment (start 75.692 48.26) (end 76.2 48.768) (width 0.508) (layer "B.Cu") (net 18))
 (segment (start 77.47 52.962) (end 77.848 52.962) (width 0.508) (layer "B.Cu") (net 18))
 (segment (start 67.31 35.555) (end 72.395 40.64) (width 0.508) (layer "B.Cu") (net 18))
 (segment (start 56.105 46.99) (end 53.4645 44.3495) (width 0.508) (layer "B.Cu") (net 21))
 (segment (start 64.389 51.562) (end 68.45 51.562) (width 0.508) (layer "B.Cu") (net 21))
 (segment (start 53.4645 44.3495) (end 53.4645 44.3205) (width 0.508) (layer "B.Cu") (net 21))
 (segment (start 62.23 35.555) (end 53.4645 44.3205) (width 0.508) (layer "B.Cu") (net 21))
 (segment (start 52.349114 53.092) (end 62.859 53.092) (width 0.508) (layer "B.Cu") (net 21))
 (segment (start 51.307 46.478) (end 51.307 52.049886) (width 0.508) (layer "B.Cu") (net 21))
 (segment (start 62.859 53.092) (end 64.389 51.562) (width 0.508) (layer "B.Cu") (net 21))
 (segment (start 51.307 52.049886) (end 52.349114 53.092) (width 0.508) (layer "B.Cu") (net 21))
 (segment (start 68.45 51.562) (end 69.85 52.962) (width 0.508) (layer "B.Cu") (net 21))
 (segment (start 53.4645 44.3205) (end 51.307 46.478) (width 0.508) (layer "B.Cu") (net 21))
 (segment (start 71.159 44.997) (end 64.052 44.997) (width 0.508) (layer "B.Cu") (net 20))
 (segment (start 74.418988 56.006) (end 75.520732 56.006) (width 0.508) (layer "B.Cu") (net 20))
 (segment (start 72.39 46.228) (end 71.159 44.997) (width 0.508) (layer "B.Cu") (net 20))
 (segment (start 66.548 54.131) (end 67.285 54.868) (width 0.508) (layer "B.Cu") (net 20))
 (segment (start 76.2 56.685268) (end 76.2 57.912) (width 0.508) (layer "B.Cu") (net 20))
 (segment (start 75.520732 56.006) (end 76.2 56.685268) (width 0.508) (layer "B.Cu") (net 20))
 (segment (start 72.39 52.962) (end 72.39 54.868) (width 0.508) (layer "B.Cu") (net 20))
 (segment (start 72.39 54.868) (end 73.280988 54.868) (width 0.508) (layer "B.Cu") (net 20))
 (segment (start 73.280988 54.868) (end 74.418988 56.006) (width 0.508) (layer "B.Cu") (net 20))
 (segment (start 64.052 44.997) (end 62.23 43.175) (width 0.508) (layer "B.Cu") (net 20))
 (segment (start 67.285 54.868) (end 72.39 54.868) (width 0.508) (layer "B.Cu") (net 20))
 (segment (start 76.2 57.912) (end 77.47 57.912) (width 0.508) (layer "B.Cu") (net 20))
 (segment (start 72.39 52.962) (end 72.39 46.228) (width 0.508) (layer "B.Cu") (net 20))
 (segment (start 69.85 57.912) (end 69.85 60.706) (width 0.508) (layer "B.Cu") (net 16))
 (segment (start 62.738 57.912) (end 69.85 57.912) (width 0.508) (layer "B.Cu") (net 16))
 (segment (start 69.85 60.706) (end 68.707 61.849) (width 0.508) (layer "B.Cu") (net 16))
 (segment (start 58.166 51.313) (end 61.717 51.313) (width 0.508) (layer "B.Cu") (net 23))
 (segment (start 61.717 51.313) (end 62.738 50.292) (width 0.508) (layer "B.Cu") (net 23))
 (segment (start 40.894 51.308) (end 41.91 52.324) (width 0.508) (layer "B.Cu") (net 3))
 (segment (start 28.956 51.308) (end 40.894 51.308) (width 0.508) (layer "B.Cu") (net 3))
 (segment (start 41.91 52.324) (end 41.91 59.436) (width 0.508) (layer "B.Cu") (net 3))
 (segment (start 37.592 58.42) (end 42.164 62.992) (width 0.508) (layer "B.Cu") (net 1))
 (segment (start 37.592 53.848) (end 37.592 58.42) (width 0.508) (layer "B.Cu") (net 1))
 (segment (start 52.102 29.313583) (end 47.633583 33.782) (width 0.508) (layer "B.Cu") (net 10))
 (segment (start 47.633583 33.782) (end 45.466 33.782) (width 0.508) (layer "B.Cu") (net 10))
 (segment (start 44.196 41.5125) (end 46.1175 43.434) (width 0.508) (layer "B.Cu") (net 10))
 (segment (start 45.466 33.782) (end 44.196 35.052) (width 0.508) (layer "B.Cu") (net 10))
 (segment (start 52.102 28.162) (end 52.102 29.313583) (width 0.508) (layer "B.Cu") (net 10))
 (segment (start 44.196 35.052) (end 44.196 41.5125) (width 0.508) (layer "B.Cu") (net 10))
 (segment (start 74.93 57.912) (end 74.93 59.138732) (width 0.508) (layer "B.Cu") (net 17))
 (segment (start 74.93 59.138732) (end 76.497268 60.706) (width 0.508) (layer "B.Cu") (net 17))
 (segment (start 76.497268 60.706) (end 76.497268 61.003268) (width 0.508) (layer "B.Cu") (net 17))
 (segment (start 76.497268 60.706) (end 80.264 60.706) (width 0.508) (layer "B.Cu") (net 17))
 (segment (start 76.497268 61.003268) (end 76.454 61.046536) (width 0.508) (layer "B.Cu") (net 17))
 (segment (start 76.454 61.046536) (end 76.454 63.627) (width 0.508) (layer "B.Cu") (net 17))
 (segment (start 87.524 50.546) (end 83.566 50.546) (width 0.508) (layer "B.Cu") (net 22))
 (segment (start 74.93 52.962) (end 74.93 54.188732) (width 0.508) (layer "B.Cu") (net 22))
 (segment (start 75.609268 54.868) (end 79.244 54.868) (width 0.508) (layer "B.Cu") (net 22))
 (segment (start 79.244 54.868) (end 83.566 50.546) (width 0.508) (layer "B.Cu") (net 22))
 (segment (start 74.93 54.188732) (end 75.609268 54.868) (width 0.508) (layer "B.Cu") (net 22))
 (segment (start 69.088 47.752) (end 59.187 47.752) (width 0.508) (layer "B.Cu") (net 25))
 (segment (start 71.12 49.784) (end 69.088 47.752) (width 0.508) (layer "B.Cu") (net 25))
 (segment (start 71.12 52.962) (end 71.12 49.784) (width 0.508) (layer "B.Cu") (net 25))
 (segment (start 59.187 47.752) (end 55.626 51.313) (width 0.508) (layer "B.Cu") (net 25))
 (segment (start 71.12 56.685268) (end 71.12 57.912) (width 0.508) (layer "B.Cu") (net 4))
 (segment (start 55.5 56.006) (end 70.440732 56.006) (width 0.508) (layer "B.Cu") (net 4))
 (segment (start 52.07 59.436) (end 55.5 56.006) (width 0.508) (layer "B.Cu") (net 4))
 (segment (start 71.12 57.912) (end 71.12 61.722) (width 0.508) (layer "B.Cu") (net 4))
 (segment (start 70.440732 56.006) (end 71.12 56.685268) (width 0.508) (layer "B.Cu") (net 4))
 (segment (start 71.12 61.722) (end 71.247 61.849) (width 0.508) (layer "B.Cu") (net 4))
 (segment (start 52.959 63.627) (end 52.324 62.992) (width 0.508) (layer "B.Cu") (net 2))
 (segment (start 72.39 57.912) (end 72.39 60.366256) (width 0.508) (layer "B.Cu") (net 2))
 (segment (start 65.786 63.627) (end 52.959 63.627) (width 0.508) (layer "B.Cu") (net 2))
 (segment (start 73.406 62.736) (end 72.515 63.627) (width 0.508) (layer "B.Cu") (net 2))
 (segment (start 72.39 60.366256) (end 73.406 61.382256) (width 0.508) (layer "B.Cu") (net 2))
 (segment (start 72.515 63.627) (end 65.786 63.627) (width 0.508) (layer "B.Cu") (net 2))
 (segment (start 73.406 61.382256) (end 73.406 62.736) (width 0.508) (layer "B.Cu") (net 2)))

